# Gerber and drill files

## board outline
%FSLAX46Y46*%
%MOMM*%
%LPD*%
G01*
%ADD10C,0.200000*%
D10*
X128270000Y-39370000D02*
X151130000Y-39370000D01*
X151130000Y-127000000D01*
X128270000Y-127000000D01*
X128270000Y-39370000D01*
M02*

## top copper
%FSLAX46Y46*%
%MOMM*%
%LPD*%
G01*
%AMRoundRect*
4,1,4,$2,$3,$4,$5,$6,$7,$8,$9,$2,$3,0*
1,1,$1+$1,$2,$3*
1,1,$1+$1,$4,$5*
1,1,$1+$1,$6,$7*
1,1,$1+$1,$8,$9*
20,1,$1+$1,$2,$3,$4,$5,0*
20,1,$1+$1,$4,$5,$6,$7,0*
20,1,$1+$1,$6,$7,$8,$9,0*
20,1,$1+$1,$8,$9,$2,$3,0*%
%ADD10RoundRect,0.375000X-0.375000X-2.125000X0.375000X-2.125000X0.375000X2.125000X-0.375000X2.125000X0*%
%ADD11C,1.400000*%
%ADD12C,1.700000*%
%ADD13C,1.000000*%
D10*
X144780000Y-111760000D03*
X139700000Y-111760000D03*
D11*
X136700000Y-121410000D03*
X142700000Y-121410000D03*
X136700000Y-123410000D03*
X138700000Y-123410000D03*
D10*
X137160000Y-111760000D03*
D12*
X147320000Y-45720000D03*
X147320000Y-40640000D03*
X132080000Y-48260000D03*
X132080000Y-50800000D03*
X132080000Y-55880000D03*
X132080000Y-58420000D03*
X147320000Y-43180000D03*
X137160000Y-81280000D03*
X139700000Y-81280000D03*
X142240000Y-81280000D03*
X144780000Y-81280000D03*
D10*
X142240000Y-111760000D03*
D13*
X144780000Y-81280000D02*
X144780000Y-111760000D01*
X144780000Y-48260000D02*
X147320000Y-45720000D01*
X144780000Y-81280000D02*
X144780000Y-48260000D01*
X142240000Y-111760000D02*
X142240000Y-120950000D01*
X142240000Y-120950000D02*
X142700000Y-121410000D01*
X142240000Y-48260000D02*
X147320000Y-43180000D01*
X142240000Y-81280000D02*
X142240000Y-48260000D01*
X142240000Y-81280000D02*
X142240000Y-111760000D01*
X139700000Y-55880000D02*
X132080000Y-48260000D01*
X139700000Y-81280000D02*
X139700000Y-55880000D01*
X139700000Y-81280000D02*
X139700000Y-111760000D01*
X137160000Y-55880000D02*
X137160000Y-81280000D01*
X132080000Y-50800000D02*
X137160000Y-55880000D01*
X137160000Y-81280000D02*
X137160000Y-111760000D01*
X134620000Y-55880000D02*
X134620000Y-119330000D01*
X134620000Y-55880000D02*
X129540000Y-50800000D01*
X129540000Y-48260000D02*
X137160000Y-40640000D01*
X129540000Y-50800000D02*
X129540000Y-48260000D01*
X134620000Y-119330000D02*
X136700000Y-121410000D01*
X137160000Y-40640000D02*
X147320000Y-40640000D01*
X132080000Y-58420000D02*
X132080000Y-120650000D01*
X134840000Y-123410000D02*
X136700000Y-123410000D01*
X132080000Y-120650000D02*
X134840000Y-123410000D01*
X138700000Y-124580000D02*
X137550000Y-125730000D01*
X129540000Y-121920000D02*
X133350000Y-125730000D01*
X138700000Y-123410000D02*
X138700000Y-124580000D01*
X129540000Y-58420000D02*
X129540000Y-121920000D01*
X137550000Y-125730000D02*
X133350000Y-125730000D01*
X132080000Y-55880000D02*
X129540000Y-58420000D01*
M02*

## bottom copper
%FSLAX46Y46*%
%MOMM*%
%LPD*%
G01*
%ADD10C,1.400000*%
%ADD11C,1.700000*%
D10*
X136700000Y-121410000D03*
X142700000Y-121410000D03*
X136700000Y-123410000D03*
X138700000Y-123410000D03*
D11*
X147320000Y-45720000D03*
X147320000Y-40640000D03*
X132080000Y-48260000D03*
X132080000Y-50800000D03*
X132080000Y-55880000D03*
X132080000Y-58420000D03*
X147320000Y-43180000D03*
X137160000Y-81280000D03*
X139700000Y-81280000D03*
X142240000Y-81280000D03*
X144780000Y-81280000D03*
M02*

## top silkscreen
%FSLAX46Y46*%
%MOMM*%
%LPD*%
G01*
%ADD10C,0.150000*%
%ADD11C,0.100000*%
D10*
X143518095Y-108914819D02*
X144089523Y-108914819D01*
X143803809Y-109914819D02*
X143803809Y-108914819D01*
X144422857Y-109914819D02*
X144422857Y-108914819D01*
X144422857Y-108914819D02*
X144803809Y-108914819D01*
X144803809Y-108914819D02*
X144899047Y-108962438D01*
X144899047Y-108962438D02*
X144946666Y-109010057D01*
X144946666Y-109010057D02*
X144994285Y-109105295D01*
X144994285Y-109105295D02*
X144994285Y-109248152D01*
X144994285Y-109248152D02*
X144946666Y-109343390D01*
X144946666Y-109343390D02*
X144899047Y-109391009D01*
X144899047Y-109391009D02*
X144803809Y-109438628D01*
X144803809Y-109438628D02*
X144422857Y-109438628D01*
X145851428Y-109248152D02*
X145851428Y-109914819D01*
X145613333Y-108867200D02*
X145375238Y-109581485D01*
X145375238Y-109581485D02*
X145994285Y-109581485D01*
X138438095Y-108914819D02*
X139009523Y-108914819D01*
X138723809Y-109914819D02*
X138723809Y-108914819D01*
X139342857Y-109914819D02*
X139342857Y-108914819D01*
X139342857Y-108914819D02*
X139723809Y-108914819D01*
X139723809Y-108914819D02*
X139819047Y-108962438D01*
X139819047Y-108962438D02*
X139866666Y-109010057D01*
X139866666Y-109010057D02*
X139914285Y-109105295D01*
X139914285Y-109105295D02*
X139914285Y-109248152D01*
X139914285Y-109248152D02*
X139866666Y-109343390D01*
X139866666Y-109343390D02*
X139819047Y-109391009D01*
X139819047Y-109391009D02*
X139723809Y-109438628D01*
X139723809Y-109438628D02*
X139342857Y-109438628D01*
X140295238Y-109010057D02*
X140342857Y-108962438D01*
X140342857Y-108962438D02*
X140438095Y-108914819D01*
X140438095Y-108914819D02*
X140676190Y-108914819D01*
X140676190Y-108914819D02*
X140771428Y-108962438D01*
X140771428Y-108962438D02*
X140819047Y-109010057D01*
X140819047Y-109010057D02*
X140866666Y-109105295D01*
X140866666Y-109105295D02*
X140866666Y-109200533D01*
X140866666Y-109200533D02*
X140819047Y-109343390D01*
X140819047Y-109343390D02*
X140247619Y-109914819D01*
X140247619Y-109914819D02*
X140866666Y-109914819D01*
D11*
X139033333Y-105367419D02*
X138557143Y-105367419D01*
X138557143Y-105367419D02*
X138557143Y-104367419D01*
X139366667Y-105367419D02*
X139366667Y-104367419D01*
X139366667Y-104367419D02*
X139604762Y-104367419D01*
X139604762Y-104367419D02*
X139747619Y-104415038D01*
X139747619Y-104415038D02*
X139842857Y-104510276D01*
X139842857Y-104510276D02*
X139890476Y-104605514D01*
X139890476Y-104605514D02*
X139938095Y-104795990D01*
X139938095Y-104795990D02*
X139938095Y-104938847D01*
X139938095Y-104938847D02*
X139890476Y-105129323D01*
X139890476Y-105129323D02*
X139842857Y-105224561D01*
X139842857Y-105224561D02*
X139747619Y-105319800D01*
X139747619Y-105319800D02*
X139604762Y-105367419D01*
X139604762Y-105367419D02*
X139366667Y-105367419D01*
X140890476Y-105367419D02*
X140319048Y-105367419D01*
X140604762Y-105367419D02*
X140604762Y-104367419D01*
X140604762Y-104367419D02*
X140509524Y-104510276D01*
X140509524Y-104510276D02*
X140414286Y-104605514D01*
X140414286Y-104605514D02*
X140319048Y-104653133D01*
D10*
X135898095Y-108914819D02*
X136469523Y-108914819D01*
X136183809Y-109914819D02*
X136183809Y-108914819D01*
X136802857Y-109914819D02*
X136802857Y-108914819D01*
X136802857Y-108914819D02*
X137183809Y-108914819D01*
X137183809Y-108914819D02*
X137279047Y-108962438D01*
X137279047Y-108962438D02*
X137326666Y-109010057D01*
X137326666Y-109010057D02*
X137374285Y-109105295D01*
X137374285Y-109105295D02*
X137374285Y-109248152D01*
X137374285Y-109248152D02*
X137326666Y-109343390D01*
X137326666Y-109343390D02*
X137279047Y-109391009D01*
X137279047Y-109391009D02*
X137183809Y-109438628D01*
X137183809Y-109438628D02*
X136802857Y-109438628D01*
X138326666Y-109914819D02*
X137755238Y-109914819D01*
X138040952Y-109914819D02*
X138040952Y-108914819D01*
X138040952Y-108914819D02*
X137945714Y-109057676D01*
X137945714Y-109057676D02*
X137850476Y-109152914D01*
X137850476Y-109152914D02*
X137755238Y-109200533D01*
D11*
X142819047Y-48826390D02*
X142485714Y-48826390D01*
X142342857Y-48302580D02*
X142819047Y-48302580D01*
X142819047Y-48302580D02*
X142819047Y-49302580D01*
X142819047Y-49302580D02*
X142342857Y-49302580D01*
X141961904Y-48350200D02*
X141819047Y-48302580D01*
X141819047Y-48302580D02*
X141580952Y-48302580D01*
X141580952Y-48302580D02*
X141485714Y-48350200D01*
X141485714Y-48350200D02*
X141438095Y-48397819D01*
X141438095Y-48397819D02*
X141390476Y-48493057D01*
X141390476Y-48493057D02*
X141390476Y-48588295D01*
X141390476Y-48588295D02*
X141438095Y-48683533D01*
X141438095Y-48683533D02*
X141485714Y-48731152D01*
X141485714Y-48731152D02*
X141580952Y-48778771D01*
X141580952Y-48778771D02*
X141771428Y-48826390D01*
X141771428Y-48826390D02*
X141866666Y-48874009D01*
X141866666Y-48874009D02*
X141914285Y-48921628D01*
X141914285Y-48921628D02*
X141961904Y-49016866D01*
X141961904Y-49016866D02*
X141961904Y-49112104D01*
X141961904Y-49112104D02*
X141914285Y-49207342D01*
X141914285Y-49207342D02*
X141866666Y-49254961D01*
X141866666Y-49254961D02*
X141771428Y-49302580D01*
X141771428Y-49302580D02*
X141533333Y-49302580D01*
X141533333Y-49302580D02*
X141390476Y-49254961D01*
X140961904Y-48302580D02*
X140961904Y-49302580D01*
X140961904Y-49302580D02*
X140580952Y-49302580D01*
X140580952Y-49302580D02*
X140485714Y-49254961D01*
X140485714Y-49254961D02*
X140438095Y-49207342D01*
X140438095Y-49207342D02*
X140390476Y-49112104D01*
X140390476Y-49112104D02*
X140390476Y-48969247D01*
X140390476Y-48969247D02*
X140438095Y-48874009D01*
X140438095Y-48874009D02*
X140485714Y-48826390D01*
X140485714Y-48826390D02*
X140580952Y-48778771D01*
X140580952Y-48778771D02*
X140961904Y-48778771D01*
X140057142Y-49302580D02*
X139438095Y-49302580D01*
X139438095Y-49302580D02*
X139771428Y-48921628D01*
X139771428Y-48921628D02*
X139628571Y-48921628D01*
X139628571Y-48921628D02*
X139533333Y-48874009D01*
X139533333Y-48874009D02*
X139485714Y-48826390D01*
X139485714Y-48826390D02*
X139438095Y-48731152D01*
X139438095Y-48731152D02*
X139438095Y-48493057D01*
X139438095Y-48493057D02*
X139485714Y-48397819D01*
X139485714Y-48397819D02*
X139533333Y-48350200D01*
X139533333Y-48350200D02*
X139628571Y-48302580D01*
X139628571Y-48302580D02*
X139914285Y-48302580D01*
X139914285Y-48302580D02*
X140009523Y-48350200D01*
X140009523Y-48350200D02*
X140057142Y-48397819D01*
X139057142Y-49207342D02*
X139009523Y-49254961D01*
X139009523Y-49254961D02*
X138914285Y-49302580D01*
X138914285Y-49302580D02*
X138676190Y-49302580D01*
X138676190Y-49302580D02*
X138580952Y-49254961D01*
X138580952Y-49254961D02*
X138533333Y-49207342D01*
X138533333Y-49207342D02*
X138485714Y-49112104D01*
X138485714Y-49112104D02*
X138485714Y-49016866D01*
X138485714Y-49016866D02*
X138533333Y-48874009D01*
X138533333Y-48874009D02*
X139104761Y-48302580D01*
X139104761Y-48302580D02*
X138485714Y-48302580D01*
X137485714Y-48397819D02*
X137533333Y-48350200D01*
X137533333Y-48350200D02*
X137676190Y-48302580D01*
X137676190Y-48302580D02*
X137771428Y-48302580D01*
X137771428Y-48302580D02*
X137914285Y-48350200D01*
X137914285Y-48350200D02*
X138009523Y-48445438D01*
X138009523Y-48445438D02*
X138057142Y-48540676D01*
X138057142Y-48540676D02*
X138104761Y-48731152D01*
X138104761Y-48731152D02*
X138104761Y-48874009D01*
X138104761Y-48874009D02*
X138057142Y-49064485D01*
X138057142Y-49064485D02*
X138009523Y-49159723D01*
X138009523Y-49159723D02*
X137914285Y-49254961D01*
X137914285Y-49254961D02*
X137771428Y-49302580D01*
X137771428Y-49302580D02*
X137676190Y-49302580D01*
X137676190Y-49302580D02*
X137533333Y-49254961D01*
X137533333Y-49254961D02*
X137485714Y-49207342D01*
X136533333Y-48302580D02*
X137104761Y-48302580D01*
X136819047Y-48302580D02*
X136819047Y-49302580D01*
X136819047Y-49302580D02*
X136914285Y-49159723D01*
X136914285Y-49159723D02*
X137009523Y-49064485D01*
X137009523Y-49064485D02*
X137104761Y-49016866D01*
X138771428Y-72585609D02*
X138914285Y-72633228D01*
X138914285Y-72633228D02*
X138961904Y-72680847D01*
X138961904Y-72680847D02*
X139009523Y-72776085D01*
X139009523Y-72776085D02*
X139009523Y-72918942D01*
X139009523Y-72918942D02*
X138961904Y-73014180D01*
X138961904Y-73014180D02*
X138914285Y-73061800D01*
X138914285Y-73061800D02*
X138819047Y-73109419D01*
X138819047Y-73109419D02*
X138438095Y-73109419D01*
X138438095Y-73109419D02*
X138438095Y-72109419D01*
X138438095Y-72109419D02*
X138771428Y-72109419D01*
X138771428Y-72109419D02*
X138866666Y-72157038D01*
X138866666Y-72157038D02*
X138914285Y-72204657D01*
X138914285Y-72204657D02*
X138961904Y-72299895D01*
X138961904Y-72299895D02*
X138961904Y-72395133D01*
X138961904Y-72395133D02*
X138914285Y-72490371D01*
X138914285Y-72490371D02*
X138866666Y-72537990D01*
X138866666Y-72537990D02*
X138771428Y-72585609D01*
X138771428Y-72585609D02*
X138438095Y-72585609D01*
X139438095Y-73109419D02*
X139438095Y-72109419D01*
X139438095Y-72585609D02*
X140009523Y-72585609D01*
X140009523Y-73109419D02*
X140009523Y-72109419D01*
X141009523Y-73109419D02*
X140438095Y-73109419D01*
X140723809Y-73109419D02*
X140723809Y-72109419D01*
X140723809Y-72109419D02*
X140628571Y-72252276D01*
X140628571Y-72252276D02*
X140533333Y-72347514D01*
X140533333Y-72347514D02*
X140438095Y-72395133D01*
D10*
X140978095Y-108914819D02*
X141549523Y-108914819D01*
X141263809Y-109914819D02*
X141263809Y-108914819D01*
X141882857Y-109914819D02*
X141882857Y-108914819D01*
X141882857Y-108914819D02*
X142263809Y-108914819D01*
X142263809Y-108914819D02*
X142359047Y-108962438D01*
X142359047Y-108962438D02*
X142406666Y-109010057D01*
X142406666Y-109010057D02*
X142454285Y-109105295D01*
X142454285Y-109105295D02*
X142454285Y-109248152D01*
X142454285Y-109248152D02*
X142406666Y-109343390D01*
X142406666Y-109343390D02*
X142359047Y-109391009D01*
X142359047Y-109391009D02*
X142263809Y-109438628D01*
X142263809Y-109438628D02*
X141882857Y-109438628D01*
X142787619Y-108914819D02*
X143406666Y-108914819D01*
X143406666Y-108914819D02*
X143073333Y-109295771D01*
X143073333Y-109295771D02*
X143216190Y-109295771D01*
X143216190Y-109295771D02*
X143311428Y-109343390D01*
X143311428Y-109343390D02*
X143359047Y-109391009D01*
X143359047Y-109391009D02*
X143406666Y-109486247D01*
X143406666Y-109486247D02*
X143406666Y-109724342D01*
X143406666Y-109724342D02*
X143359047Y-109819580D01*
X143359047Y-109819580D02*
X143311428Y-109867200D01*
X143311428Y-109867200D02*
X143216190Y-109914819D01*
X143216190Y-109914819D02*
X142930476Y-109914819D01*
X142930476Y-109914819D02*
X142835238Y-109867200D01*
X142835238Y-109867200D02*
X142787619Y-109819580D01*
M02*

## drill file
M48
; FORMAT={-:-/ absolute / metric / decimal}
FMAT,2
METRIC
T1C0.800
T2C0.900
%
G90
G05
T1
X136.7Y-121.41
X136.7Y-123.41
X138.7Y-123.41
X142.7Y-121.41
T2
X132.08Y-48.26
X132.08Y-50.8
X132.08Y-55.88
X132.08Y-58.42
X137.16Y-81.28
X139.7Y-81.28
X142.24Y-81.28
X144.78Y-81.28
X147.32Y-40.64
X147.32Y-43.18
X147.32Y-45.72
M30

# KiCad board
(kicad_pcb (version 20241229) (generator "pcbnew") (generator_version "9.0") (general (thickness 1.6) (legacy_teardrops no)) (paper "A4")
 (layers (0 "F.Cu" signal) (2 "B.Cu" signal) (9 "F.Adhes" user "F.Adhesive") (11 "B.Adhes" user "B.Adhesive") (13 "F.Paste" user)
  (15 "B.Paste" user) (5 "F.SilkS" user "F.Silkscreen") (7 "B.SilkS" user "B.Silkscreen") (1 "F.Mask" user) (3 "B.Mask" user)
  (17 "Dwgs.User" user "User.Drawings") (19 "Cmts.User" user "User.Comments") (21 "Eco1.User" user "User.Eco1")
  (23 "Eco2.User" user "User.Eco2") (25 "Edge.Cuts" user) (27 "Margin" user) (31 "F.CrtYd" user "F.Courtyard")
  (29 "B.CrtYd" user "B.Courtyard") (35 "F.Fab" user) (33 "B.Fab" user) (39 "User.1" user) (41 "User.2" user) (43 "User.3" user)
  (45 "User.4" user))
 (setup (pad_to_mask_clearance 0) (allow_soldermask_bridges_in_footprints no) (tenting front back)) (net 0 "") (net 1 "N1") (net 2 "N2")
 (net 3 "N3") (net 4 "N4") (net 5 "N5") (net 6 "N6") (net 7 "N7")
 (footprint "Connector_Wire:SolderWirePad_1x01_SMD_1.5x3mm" (layer "F.Cu") (at 144.78 111.76)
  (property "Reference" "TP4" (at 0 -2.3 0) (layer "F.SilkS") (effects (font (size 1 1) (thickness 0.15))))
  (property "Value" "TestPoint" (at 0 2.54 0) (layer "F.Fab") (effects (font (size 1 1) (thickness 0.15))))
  (pad "1" smd roundrect (at 0 0) (size 1.5 5) (layers "F.Cu" "F.Mask") (roundrect_rratio 0.25) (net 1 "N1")))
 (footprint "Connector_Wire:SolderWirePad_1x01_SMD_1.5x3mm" (layer "F.Cu") (at 139.7 111.76)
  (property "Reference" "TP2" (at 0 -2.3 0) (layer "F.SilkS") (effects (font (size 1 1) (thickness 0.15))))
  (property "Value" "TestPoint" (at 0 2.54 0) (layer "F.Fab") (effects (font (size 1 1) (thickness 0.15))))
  (pad "1" smd roundrect (at 0 0) (size 1.5 5) (layers "F.Cu" "F.Mask") (roundrect_rratio 0.25) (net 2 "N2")))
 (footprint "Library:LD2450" (layer "F.Cu") (at 139.7 105.41)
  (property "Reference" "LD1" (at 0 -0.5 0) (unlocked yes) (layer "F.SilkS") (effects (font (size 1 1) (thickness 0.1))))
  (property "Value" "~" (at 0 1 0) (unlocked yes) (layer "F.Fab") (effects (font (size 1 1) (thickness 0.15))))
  (pad "1" thru_hole circle (at -3 16 90) (size 1.4 1.4) (drill 0.8) (layers "*.Cu" "*.Mask") (remove_unused_layers yes)
   (keep_end_layers yes) (zone_layer_connections) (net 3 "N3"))
  (pad "2" thru_hole circle (at 3 16 90) (size 1.4 1.4) (drill 0.8) (layers "*.Cu" "*.Mask") (remove_unused_layers yes)
   (keep_end_layers yes) (zone_layer_connections) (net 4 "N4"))
  (pad "3" thru_hole circle (at -3 18 90) (size 1.4 1.4) (drill 0.8) (layers "*.Cu" "*.Mask") (remove_unused_layers yes)
   (keep_end_layers yes) (zone_layer_connections) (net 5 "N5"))
  (pad "4" thru_hole circle (at -1 18 90) (size 1.4 1.4) (drill 0.8) (layers "*.Cu" "*.Mask") (remove_unused_layers yes)
   (keep_end_layers yes) (zone_layer_connections) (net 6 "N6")))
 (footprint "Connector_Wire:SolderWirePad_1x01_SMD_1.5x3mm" (layer "F.Cu") (at 137.16 111.76)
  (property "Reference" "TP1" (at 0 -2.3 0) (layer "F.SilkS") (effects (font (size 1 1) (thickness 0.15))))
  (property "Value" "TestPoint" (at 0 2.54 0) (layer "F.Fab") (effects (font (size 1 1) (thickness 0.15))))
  (pad "1" smd roundrect (at 0 0) (size 1.5 5) (layers "F.Cu" "F.Mask") (roundrect_rratio 0.25) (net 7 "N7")))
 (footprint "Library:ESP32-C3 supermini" (layer "F.Cu") (at 139.7 50.8 180)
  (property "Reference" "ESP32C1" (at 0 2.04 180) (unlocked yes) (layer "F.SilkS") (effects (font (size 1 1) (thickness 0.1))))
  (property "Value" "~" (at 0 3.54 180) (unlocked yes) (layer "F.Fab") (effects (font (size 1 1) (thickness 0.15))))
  (pad "3.3V" thru_hole circle (at -7.62 5.08 180) (size 1.7 1.7) (drill 0.9) (layers "*.Cu" "*.Mask") (remove_unused_layers yes)
   (keep_end_layers yes) (zone_layer_connections) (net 1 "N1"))
  (pad "5V" thru_hole circle (at -7.62 10.16 180) (size 1.7 1.7) (drill 0.9) (layers "*.Cu" "*.Mask") (remove_unused_layers yes)
   (keep_end_layers yes) (zone_layer_connections) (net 3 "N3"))
  (pad "8" thru_hole circle (at 7.62 2.54 180) (size 1.7 1.7) (drill 0.9) (layers "*.Cu" "*.Mask") (remove_unused_layers yes)
   (keep_end_layers yes) (zone_layer_connections) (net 2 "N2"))
  (pad "9" thru_hole circle (at 7.62 0 180) (size 1.7 1.7) (drill 0.9) (layers "*.Cu" "*.Mask") (remove_unused_layers yes)
   (keep_end_layers yes) (zone_layer_connections) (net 7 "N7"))
  (pad "20" thru_hole circle (at 7.62 -5.08 180) (size 1.7 1.7) (drill 0.9) (layers "*.Cu" "*.Mask") (remove_unused_layers yes)
   (keep_end_layers yes) (zone_layer_connections) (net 6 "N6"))
  (pad "21" thru_hole circle (at 7.62 -7.62 180) (size 1.7 1.7) (drill 0.9) (layers "*.Cu" "*.Mask") (remove_unused_layers yes)
   (keep_end_layers yes) (zone_layer_connections) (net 5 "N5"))
  (pad "GND" thru_hole circle (at -7.62 7.62 180) (size 1.7 1.7) (drill 0.9) (layers "*.Cu" "*.Mask") (remove_unused_layers yes)
   (keep_end_layers yes) (zone_layer_connections) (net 4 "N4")))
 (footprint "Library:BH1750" (layer "F.Cu") (at 139.7 73.152)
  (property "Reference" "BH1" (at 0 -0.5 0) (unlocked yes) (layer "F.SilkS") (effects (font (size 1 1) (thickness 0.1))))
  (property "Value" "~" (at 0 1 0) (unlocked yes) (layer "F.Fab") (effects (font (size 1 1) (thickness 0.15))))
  (pad "1" thru_hole circle (at -2.54 8.128 90) (size 1.7 1.7) (drill 0.9) (layers "*.Cu" "*.Mask") (remove_unused_layers yes)
   (keep_end_layers yes) (zone_layer_connections) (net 7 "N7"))
  (pad "2" thru_hole circle (at 0 8.128 90) (size 1.7 1.7) (drill 0.9) (layers "*.Cu" "*.Mask") (remove_unused_layers yes)
   (keep_end_layers yes) (zone_layer_connections) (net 2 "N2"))
  (pad "3" thru_hole circle (at 2.54 8.128 90) (size 1.7 1.7) (drill 0.9) (layers "*.Cu" "*.Mask") (remove_unused_layers yes)
   (keep_end_layers yes) (zone_layer_connections) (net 4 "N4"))
  (pad "4" thru_hole circle (at 5.08 8.128 90) (size 1.7 1.7) (drill 0.9) (layers "*.Cu" "*.Mask") (remove_unused_layers yes)
   (keep_end_layers yes) (zone_layer_connections) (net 1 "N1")))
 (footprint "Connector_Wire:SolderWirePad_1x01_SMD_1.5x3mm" (layer "F.Cu") (at 142.24 111.76)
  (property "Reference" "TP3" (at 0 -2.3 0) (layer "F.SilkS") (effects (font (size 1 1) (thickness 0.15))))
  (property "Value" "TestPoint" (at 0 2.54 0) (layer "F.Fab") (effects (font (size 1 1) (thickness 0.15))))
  (pad "1" smd roundrect (at 0 0) (size 1.5 5) (layers "F.Cu" "F.Mask") (roundrect_rratio 0.25) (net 4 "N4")))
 (gr_rect (start 128.27 39.37) (end 151.13 127) (stroke (width 0.2) (type solid)) (fill no) (layer "Edge.Cuts"))
 (segment (start 144.78 81.28) (end 144.78 111.76) (width 1) (layer "F.Cu") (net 1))
 (segment (start 144.78 48.26) (end 147.32 45.72) (width 1) (layer "F.Cu") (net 1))
 (segment (start 144.78 81.28) (end 144.78 48.26) (width 1) (layer "F.Cu") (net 1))
 (segment (start 142.24 111.76) (end 142.24 120.95) (width 1) (layer "F.Cu") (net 4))
 (segment (start 142.24 120.95) (end 142.7 121.41) (width 1) (layer "F.Cu") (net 4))
 (segment (start 142.24 48.26) (end 147.32 43.18) (width 1) (layer "F.Cu") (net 4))
 (segment (start 142.24 81.28) (end 142.24 48.26) (width 1) (layer "F.Cu") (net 4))
 (segment (start 142.24 81.28) (end 142.24 111.76) (width 1) (layer "F.Cu") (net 4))
 (segment (start 139.7 55.88) (end 132.08 48.26) (width 1) (layer "F.Cu") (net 2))
 (segment (start 139.7 81.28) (end 139.7 55.88) (width 1) (layer "F.Cu") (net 2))
 (segment (start 139.7 81.28) (end 139.7 111.76) (width 1) (layer "F.Cu") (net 2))
 (segment (start 137.16 55.88) (end 137.16 81.28) (width 1) (layer "F.Cu") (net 7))
 (segment (start 132.08 50.8) (end 137.16 55.88) (width 1) (layer "F.Cu") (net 7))
 (segment (start 137.16 81.28) (end 137.16 111.76) (width 1) (layer "F.Cu") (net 7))
 (segment (start 134.62 55.88) (end 134.62 119.33) (width 1) (layer "F.Cu") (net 3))
 (segment (start 134.62 55.88) (end 129.54 50.8) (width 1) (layer "F.Cu") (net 3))
 (segment (start 129.54 48.26) (end 137.16 40.64) (width 1) (layer "F.Cu") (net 3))
 (segment (start 129.54 50.8) (end 129.54 48.26) (width 1) (layer "F.Cu") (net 3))
 (segment (start 134.62 119.33) (end 136.7 121.41) (width 1) (layer "F.Cu") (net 3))
 (segment (start 137.16 40.64) (end 147.32 40.64) (width 1) (layer "F.Cu") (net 3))
 (segment (start 132.08 58.42) (end 132.08 120.65) (width 1) (layer "F.Cu") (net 5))
 (segment (start 134.84 123.41) (end 136.7 123.41) (width 1) (layer "F.Cu") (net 5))
 (segment (start 132.08 120.65) (end 134.84 123.41) (width 1) (layer "F.Cu") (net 5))
 (segment (start 138.7 124.58) (end 137.55 125.73) (width 1) (layer "F.Cu") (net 6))
 (segment (start 129.54 121.92) (end 133.35 125.73) (width 1) (layer "F.Cu") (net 6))
 (segment (start 138.7 123.41) (end 138.7 124.58) (width 1) (layer "F.Cu") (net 6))
 (segment (start 129.54 58.42) (end 129.54 121.92) (width 1) (layer "F.Cu") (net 6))
 (segment (start 137.55 125.73) (end 133.35 125.73) (width 1) (layer "F.Cu") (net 6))
 (segment (start 132.08 55.88) (end 129.54 58.42) (width 1) (layer "F.Cu") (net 6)))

